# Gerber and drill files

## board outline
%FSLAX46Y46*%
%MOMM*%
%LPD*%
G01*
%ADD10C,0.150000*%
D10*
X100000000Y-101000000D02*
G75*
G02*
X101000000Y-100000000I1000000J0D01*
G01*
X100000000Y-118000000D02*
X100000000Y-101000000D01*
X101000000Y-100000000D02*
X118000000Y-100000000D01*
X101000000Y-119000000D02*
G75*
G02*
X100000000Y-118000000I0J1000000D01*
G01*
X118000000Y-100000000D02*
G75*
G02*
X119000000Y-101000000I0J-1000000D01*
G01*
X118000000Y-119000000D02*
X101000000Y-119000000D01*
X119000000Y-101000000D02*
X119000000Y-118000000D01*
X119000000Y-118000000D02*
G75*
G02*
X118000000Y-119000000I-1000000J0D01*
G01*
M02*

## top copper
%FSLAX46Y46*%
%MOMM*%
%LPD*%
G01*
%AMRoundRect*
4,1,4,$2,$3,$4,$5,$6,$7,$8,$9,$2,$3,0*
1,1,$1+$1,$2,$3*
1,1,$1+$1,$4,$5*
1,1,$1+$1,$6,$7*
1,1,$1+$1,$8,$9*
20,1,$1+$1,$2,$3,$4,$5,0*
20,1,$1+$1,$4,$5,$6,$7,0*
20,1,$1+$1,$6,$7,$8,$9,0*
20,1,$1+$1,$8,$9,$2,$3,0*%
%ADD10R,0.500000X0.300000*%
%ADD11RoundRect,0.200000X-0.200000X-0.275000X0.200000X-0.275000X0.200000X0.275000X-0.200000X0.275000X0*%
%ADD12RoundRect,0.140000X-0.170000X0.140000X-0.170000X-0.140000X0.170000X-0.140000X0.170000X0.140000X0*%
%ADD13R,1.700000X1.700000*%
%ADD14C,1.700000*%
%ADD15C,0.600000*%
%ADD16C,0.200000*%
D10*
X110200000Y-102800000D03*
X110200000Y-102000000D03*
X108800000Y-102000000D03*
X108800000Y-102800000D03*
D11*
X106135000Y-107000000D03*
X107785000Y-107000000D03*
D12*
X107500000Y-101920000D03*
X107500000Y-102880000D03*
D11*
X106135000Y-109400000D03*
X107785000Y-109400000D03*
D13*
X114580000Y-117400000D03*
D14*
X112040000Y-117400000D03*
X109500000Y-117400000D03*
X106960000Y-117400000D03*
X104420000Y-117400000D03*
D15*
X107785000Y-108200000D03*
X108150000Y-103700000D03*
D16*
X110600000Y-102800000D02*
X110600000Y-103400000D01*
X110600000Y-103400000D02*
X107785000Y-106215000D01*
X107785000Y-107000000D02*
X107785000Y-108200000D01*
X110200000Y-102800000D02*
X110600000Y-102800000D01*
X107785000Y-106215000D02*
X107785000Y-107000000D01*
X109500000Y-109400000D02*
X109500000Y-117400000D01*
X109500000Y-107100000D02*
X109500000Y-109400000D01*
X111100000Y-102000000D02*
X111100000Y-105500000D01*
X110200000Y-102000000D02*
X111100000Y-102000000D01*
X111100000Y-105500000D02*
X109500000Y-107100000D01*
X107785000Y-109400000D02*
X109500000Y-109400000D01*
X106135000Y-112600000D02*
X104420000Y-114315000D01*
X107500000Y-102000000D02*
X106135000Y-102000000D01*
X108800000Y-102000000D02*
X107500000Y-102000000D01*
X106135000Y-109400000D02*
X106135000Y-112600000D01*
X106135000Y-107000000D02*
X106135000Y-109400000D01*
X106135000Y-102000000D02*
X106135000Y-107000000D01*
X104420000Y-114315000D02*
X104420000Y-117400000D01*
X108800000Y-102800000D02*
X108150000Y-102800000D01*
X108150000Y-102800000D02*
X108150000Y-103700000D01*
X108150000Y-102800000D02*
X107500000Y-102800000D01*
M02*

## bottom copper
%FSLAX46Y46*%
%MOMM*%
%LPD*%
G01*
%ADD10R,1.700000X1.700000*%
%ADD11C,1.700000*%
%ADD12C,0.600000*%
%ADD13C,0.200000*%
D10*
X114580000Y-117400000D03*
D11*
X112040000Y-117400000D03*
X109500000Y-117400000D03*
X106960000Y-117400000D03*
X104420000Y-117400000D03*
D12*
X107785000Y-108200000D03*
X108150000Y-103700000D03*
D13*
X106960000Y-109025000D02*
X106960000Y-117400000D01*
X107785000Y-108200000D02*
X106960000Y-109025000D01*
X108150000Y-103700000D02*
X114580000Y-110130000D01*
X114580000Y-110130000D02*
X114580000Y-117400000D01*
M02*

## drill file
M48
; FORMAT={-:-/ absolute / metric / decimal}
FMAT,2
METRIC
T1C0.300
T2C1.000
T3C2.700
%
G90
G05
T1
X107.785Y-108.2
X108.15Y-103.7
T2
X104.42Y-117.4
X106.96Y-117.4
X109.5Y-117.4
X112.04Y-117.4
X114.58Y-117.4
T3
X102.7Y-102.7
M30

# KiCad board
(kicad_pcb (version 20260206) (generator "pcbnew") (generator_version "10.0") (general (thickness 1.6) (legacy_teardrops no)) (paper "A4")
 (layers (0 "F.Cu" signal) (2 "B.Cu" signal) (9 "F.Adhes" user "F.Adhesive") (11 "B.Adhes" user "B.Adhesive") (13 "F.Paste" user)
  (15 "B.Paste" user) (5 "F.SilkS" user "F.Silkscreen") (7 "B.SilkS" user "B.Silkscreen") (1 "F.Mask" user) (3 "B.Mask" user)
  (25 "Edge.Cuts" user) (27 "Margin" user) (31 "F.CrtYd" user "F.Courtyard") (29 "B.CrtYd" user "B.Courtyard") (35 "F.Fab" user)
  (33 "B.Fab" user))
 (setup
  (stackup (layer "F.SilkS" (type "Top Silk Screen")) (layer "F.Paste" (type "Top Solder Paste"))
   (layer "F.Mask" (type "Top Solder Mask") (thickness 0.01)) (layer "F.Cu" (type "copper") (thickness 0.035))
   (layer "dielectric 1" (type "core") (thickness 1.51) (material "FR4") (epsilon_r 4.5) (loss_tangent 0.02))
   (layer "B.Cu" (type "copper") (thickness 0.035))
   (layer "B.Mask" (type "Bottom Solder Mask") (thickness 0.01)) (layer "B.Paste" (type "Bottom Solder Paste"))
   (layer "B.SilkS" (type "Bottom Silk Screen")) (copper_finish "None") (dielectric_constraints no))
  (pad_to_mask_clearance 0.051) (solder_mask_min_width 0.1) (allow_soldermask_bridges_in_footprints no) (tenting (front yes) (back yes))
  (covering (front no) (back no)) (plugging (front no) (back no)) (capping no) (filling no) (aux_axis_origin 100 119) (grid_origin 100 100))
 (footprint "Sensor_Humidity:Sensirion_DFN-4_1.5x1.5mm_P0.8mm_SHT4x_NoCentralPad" (layer "F.Cu") (at 109.5 102.4 180)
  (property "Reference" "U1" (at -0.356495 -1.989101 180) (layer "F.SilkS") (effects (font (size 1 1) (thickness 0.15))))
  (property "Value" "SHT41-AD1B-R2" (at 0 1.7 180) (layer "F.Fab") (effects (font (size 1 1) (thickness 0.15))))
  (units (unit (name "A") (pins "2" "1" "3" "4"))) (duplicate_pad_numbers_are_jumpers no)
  (pad "1" smd rect (at -0.7 -0.4 180) (size 0.5 0.3) (layers "F.Cu" "F.Mask" "F.Paste") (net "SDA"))
  (pad "2" smd rect (at -0.7 0.4 180) (size 0.5 0.3) (layers "F.Cu" "F.Mask" "F.Paste") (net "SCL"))
  (pad "3" smd rect (at 0.7 0.4 180) (size 0.5 0.3) (layers "F.Cu" "F.Mask" "F.Paste") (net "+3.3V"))
  (pad "4" smd rect (at 0.7 -0.4 180) (size 0.5 0.3) (layers "F.Cu" "F.Mask" "F.Paste") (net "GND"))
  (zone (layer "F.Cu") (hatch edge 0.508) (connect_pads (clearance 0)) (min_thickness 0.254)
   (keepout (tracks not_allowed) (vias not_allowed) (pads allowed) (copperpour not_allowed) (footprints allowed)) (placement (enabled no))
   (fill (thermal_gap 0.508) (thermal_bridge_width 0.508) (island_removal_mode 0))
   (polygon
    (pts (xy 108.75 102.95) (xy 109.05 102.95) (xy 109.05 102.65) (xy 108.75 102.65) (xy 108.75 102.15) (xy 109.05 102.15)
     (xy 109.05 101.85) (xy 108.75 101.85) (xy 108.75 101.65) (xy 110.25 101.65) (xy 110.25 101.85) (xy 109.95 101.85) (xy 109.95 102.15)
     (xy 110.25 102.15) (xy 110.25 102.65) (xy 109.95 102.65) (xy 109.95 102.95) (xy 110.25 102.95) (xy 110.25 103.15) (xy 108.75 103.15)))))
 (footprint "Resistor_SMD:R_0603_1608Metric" (layer "F.Cu") (at 106.96 107)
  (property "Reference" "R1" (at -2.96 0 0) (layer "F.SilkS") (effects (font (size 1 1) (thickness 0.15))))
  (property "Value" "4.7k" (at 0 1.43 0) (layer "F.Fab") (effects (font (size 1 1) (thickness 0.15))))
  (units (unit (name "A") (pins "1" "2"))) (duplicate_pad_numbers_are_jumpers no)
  (pad "1" smd roundrect (at -0.825 0) (size 0.8 0.95) (layers "F.Cu" "F.Mask" "F.Paste") (roundrect_rratio 0.25) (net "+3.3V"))
  (pad "2" smd roundrect (at 0.825 0) (size 0.8 0.95) (layers "F.Cu" "F.Mask" "F.Paste") (roundrect_rratio 0.25) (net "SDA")))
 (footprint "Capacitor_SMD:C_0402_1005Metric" (layer "F.Cu") (at 107.5 102.4 -90)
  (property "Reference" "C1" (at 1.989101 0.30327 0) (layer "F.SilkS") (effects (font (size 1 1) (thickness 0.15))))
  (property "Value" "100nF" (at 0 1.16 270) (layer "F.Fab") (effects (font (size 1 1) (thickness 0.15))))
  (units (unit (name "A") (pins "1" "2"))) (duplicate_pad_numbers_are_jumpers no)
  (pad "1" smd roundrect (at -0.48 0 270) (size 0.56 0.62) (layers "F.Cu" "F.Mask" "F.Paste") (roundrect_rratio 0.25) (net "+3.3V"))
  (pad "2" smd roundrect (at 0.48 0 270) (size 0.56 0.62) (layers "F.Cu" "F.Mask" "F.Paste") (roundrect_rratio 0.25) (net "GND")))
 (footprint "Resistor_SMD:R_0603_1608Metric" (layer "F.Cu") (at 106.96 109.4)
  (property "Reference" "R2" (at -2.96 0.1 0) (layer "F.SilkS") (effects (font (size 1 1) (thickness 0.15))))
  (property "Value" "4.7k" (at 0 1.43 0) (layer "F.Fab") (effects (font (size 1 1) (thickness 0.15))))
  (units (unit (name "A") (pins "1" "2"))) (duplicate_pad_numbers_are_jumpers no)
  (pad "1" smd roundrect (at -0.825 0) (size 0.8 0.95) (layers "F.Cu" "F.Mask" "F.Paste") (roundrect_rratio 0.25) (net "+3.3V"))
  (pad "2" smd roundrect (at 0.825 0) (size 0.8 0.95) (layers "F.Cu" "F.Mask" "F.Paste") (roundrect_rratio 0.25) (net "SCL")))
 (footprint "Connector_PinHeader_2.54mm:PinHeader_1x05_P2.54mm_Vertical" (layer "F.Cu") (at 114.58 117.4 -90)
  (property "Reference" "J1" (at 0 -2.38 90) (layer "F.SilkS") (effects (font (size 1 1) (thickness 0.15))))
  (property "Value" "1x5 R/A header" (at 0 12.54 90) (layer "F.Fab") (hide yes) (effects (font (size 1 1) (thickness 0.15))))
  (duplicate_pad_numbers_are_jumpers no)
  (pad "1" thru_hole rect (at 0 0 270) (size 1.7 1.7) (drill 1) (layers "*.Cu" "*.Mask") (remove_unused_layers no) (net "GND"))
  (pad "2" thru_hole circle (at 0 2.54 270) (size 1.7 1.7) (drill 1) (layers "*.Cu" "*.Mask") (remove_unused_layers no)
   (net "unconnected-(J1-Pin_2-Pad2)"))
  (pad "3" thru_hole circle (at 0 5.08 270) (size 1.7 1.7) (drill 1) (layers "*.Cu" "*.Mask") (remove_unused_layers no) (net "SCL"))
  (pad "4" thru_hole circle (at 0 7.62 270) (size 1.7 1.7) (drill 1) (layers "*.Cu" "*.Mask") (remove_unused_layers no) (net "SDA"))
  (pad "5" thru_hole circle (at 0 10.16 270) (size 1.7 1.7) (drill 1) (layers "*.Cu" "*.Mask") (remove_unused_layers no) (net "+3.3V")))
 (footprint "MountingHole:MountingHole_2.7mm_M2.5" (layer "F.Cu") (at 102.7 102.7)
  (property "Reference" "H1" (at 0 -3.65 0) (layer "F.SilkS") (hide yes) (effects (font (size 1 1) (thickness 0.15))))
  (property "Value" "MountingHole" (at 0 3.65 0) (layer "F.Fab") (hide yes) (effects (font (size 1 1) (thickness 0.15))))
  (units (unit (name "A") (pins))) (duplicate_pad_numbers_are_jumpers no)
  (pad "" np_thru_hole circle (at 0 0) (size 2.7 2.7) (drill 2.7) (layers "*.Cu" "*.Mask")))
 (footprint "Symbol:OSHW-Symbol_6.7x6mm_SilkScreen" (layer "B.Cu") (at 114.732 103.556 180)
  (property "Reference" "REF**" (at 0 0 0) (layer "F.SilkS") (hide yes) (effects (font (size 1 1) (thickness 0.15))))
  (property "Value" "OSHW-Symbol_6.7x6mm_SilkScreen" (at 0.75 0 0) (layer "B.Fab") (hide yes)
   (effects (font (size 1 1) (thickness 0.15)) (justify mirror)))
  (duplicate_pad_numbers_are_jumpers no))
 (gr_arc (start 100 101) (mid 100.292893 100.292893) (end 101 100) (stroke (width 0.15) (type default)) (layer "Edge.Cuts"))
 (gr_line (start 100 118) (end 100 101) (stroke (width 0.15) (type default)) (layer "Edge.Cuts"))
 (gr_line (start 101 100) (end 118 100) (stroke (width 0.15) (type default)) (layer "Edge.Cuts"))
 (gr_arc (start 101 119) (mid 100.292893 118.707107) (end 100 118) (stroke (width 0.15) (type default)) (layer "Edge.Cuts"))
 (gr_arc (start 118 100) (mid 118.707107 100.292893) (end 119 101) (stroke (width 0.15) (type default)) (layer "Edge.Cuts"))
 (gr_line (start 118 119) (end 101 119) (stroke (width 0.15) (type default)) (layer "Edge.Cuts"))
 (gr_line (start 119 101) (end 119 118) (stroke (width 0.15) (type default)) (layer "Edge.Cuts"))
 (gr_arc (start 119 118) (mid 118.707107 118.707107) (end 118 119) (stroke (width 0.15) (type default)) (layer "Edge.Cuts"))
 (segment (start 110.6 102.8) (end 110.6 103.4) (width 0.2) (layer "F.Cu") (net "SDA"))
 (segment (start 110.6 103.4) (end 107.785 106.215) (width 0.2) (layer "F.Cu") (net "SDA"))
 (segment (start 107.785 107) (end 107.785 108.2) (width 0.2) (layer "F.Cu") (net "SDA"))
 (segment (start 110.2 102.8) (end 110.6 102.8) (width 0.2) (layer "F.Cu") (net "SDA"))
 (segment (start 107.785 106.215) (end 107.785 107) (width 0.2) (layer "F.Cu") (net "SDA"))
 (via (at 107.785 108.2) (size 0.6) (drill 0.3) (layers "F.Cu" "B.Cu") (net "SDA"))
 (segment (start 106.96 109.025) (end 106.96 117.4) (width 0.2) (layer "B.Cu") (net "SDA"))
 (segment (start 107.785 108.2) (end 106.96 109.025) (width 0.2) (layer "B.Cu") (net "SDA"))
 (segment (start 109.5 109.4) (end 109.5 117.4) (width 0.2) (layer "F.Cu") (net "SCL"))
 (segment (start 109.5 107.1) (end 109.5 109.4) (width 0.2) (layer "F.Cu") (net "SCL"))
 (segment (start 111.1 102) (end 111.1 105.5) (width 0.2) (layer "F.Cu") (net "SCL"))
 (segment (start 110.2 102) (end 111.1 102) (width 0.2) (layer "F.Cu") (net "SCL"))
 (segment (start 111.1 105.5) (end 109.5 107.1) (width 0.2) (layer "F.Cu") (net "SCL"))
 (segment (start 107.785 109.4) (end 109.5 109.4) (width 0.2) (layer "F.Cu") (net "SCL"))
 (segment (start 106.135 112.6) (end 104.42 114.315) (width 0.2) (layer "F.Cu") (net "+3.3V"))
 (segment (start 107.5 102) (end 106.135 102) (width 0.2) (layer "F.Cu") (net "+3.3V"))
 (segment (start 108.8 102) (end 107.5 102) (width 0.2) (layer "F.Cu") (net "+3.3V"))
 (segment (start 106.135 109.4) (end 106.135 112.6) (width 0.2) (layer "F.Cu") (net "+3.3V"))
 (segment (start 106.135 107) (end 106.135 109.4) (width 0.2) (layer "F.Cu") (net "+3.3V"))
 (segment (start 106.135 102) (end 106.135 107) (width 0.2) (layer "F.Cu") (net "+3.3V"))
 (segment (start 104.42 114.315) (end 104.42 117.4) (width 0.2) (layer "F.Cu") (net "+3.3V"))
 (segment (start 108.8 102.8) (end 108.15 102.8) (width 0.2) (layer "F.Cu") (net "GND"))
 (segment (start 108.15 102.8) (end 108.15 103.7) (width 0.2) (layer "F.Cu") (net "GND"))
 (segment (start 108.15 102.8) (end 107.5 102.8) (width 0.2) (layer "F.Cu") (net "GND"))
 (via (at 108.15 103.7) (size 0.6) (drill 0.3) (layers "F.Cu" "B.Cu") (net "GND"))
 (segment (start 108.15 103.7) (end 114.58 110.13) (width 0.2) (layer "B.Cu") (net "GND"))
 (segment (start 114.58 110.13) (end 114.58 117.4) (width 0.2) (layer "B.Cu") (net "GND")))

